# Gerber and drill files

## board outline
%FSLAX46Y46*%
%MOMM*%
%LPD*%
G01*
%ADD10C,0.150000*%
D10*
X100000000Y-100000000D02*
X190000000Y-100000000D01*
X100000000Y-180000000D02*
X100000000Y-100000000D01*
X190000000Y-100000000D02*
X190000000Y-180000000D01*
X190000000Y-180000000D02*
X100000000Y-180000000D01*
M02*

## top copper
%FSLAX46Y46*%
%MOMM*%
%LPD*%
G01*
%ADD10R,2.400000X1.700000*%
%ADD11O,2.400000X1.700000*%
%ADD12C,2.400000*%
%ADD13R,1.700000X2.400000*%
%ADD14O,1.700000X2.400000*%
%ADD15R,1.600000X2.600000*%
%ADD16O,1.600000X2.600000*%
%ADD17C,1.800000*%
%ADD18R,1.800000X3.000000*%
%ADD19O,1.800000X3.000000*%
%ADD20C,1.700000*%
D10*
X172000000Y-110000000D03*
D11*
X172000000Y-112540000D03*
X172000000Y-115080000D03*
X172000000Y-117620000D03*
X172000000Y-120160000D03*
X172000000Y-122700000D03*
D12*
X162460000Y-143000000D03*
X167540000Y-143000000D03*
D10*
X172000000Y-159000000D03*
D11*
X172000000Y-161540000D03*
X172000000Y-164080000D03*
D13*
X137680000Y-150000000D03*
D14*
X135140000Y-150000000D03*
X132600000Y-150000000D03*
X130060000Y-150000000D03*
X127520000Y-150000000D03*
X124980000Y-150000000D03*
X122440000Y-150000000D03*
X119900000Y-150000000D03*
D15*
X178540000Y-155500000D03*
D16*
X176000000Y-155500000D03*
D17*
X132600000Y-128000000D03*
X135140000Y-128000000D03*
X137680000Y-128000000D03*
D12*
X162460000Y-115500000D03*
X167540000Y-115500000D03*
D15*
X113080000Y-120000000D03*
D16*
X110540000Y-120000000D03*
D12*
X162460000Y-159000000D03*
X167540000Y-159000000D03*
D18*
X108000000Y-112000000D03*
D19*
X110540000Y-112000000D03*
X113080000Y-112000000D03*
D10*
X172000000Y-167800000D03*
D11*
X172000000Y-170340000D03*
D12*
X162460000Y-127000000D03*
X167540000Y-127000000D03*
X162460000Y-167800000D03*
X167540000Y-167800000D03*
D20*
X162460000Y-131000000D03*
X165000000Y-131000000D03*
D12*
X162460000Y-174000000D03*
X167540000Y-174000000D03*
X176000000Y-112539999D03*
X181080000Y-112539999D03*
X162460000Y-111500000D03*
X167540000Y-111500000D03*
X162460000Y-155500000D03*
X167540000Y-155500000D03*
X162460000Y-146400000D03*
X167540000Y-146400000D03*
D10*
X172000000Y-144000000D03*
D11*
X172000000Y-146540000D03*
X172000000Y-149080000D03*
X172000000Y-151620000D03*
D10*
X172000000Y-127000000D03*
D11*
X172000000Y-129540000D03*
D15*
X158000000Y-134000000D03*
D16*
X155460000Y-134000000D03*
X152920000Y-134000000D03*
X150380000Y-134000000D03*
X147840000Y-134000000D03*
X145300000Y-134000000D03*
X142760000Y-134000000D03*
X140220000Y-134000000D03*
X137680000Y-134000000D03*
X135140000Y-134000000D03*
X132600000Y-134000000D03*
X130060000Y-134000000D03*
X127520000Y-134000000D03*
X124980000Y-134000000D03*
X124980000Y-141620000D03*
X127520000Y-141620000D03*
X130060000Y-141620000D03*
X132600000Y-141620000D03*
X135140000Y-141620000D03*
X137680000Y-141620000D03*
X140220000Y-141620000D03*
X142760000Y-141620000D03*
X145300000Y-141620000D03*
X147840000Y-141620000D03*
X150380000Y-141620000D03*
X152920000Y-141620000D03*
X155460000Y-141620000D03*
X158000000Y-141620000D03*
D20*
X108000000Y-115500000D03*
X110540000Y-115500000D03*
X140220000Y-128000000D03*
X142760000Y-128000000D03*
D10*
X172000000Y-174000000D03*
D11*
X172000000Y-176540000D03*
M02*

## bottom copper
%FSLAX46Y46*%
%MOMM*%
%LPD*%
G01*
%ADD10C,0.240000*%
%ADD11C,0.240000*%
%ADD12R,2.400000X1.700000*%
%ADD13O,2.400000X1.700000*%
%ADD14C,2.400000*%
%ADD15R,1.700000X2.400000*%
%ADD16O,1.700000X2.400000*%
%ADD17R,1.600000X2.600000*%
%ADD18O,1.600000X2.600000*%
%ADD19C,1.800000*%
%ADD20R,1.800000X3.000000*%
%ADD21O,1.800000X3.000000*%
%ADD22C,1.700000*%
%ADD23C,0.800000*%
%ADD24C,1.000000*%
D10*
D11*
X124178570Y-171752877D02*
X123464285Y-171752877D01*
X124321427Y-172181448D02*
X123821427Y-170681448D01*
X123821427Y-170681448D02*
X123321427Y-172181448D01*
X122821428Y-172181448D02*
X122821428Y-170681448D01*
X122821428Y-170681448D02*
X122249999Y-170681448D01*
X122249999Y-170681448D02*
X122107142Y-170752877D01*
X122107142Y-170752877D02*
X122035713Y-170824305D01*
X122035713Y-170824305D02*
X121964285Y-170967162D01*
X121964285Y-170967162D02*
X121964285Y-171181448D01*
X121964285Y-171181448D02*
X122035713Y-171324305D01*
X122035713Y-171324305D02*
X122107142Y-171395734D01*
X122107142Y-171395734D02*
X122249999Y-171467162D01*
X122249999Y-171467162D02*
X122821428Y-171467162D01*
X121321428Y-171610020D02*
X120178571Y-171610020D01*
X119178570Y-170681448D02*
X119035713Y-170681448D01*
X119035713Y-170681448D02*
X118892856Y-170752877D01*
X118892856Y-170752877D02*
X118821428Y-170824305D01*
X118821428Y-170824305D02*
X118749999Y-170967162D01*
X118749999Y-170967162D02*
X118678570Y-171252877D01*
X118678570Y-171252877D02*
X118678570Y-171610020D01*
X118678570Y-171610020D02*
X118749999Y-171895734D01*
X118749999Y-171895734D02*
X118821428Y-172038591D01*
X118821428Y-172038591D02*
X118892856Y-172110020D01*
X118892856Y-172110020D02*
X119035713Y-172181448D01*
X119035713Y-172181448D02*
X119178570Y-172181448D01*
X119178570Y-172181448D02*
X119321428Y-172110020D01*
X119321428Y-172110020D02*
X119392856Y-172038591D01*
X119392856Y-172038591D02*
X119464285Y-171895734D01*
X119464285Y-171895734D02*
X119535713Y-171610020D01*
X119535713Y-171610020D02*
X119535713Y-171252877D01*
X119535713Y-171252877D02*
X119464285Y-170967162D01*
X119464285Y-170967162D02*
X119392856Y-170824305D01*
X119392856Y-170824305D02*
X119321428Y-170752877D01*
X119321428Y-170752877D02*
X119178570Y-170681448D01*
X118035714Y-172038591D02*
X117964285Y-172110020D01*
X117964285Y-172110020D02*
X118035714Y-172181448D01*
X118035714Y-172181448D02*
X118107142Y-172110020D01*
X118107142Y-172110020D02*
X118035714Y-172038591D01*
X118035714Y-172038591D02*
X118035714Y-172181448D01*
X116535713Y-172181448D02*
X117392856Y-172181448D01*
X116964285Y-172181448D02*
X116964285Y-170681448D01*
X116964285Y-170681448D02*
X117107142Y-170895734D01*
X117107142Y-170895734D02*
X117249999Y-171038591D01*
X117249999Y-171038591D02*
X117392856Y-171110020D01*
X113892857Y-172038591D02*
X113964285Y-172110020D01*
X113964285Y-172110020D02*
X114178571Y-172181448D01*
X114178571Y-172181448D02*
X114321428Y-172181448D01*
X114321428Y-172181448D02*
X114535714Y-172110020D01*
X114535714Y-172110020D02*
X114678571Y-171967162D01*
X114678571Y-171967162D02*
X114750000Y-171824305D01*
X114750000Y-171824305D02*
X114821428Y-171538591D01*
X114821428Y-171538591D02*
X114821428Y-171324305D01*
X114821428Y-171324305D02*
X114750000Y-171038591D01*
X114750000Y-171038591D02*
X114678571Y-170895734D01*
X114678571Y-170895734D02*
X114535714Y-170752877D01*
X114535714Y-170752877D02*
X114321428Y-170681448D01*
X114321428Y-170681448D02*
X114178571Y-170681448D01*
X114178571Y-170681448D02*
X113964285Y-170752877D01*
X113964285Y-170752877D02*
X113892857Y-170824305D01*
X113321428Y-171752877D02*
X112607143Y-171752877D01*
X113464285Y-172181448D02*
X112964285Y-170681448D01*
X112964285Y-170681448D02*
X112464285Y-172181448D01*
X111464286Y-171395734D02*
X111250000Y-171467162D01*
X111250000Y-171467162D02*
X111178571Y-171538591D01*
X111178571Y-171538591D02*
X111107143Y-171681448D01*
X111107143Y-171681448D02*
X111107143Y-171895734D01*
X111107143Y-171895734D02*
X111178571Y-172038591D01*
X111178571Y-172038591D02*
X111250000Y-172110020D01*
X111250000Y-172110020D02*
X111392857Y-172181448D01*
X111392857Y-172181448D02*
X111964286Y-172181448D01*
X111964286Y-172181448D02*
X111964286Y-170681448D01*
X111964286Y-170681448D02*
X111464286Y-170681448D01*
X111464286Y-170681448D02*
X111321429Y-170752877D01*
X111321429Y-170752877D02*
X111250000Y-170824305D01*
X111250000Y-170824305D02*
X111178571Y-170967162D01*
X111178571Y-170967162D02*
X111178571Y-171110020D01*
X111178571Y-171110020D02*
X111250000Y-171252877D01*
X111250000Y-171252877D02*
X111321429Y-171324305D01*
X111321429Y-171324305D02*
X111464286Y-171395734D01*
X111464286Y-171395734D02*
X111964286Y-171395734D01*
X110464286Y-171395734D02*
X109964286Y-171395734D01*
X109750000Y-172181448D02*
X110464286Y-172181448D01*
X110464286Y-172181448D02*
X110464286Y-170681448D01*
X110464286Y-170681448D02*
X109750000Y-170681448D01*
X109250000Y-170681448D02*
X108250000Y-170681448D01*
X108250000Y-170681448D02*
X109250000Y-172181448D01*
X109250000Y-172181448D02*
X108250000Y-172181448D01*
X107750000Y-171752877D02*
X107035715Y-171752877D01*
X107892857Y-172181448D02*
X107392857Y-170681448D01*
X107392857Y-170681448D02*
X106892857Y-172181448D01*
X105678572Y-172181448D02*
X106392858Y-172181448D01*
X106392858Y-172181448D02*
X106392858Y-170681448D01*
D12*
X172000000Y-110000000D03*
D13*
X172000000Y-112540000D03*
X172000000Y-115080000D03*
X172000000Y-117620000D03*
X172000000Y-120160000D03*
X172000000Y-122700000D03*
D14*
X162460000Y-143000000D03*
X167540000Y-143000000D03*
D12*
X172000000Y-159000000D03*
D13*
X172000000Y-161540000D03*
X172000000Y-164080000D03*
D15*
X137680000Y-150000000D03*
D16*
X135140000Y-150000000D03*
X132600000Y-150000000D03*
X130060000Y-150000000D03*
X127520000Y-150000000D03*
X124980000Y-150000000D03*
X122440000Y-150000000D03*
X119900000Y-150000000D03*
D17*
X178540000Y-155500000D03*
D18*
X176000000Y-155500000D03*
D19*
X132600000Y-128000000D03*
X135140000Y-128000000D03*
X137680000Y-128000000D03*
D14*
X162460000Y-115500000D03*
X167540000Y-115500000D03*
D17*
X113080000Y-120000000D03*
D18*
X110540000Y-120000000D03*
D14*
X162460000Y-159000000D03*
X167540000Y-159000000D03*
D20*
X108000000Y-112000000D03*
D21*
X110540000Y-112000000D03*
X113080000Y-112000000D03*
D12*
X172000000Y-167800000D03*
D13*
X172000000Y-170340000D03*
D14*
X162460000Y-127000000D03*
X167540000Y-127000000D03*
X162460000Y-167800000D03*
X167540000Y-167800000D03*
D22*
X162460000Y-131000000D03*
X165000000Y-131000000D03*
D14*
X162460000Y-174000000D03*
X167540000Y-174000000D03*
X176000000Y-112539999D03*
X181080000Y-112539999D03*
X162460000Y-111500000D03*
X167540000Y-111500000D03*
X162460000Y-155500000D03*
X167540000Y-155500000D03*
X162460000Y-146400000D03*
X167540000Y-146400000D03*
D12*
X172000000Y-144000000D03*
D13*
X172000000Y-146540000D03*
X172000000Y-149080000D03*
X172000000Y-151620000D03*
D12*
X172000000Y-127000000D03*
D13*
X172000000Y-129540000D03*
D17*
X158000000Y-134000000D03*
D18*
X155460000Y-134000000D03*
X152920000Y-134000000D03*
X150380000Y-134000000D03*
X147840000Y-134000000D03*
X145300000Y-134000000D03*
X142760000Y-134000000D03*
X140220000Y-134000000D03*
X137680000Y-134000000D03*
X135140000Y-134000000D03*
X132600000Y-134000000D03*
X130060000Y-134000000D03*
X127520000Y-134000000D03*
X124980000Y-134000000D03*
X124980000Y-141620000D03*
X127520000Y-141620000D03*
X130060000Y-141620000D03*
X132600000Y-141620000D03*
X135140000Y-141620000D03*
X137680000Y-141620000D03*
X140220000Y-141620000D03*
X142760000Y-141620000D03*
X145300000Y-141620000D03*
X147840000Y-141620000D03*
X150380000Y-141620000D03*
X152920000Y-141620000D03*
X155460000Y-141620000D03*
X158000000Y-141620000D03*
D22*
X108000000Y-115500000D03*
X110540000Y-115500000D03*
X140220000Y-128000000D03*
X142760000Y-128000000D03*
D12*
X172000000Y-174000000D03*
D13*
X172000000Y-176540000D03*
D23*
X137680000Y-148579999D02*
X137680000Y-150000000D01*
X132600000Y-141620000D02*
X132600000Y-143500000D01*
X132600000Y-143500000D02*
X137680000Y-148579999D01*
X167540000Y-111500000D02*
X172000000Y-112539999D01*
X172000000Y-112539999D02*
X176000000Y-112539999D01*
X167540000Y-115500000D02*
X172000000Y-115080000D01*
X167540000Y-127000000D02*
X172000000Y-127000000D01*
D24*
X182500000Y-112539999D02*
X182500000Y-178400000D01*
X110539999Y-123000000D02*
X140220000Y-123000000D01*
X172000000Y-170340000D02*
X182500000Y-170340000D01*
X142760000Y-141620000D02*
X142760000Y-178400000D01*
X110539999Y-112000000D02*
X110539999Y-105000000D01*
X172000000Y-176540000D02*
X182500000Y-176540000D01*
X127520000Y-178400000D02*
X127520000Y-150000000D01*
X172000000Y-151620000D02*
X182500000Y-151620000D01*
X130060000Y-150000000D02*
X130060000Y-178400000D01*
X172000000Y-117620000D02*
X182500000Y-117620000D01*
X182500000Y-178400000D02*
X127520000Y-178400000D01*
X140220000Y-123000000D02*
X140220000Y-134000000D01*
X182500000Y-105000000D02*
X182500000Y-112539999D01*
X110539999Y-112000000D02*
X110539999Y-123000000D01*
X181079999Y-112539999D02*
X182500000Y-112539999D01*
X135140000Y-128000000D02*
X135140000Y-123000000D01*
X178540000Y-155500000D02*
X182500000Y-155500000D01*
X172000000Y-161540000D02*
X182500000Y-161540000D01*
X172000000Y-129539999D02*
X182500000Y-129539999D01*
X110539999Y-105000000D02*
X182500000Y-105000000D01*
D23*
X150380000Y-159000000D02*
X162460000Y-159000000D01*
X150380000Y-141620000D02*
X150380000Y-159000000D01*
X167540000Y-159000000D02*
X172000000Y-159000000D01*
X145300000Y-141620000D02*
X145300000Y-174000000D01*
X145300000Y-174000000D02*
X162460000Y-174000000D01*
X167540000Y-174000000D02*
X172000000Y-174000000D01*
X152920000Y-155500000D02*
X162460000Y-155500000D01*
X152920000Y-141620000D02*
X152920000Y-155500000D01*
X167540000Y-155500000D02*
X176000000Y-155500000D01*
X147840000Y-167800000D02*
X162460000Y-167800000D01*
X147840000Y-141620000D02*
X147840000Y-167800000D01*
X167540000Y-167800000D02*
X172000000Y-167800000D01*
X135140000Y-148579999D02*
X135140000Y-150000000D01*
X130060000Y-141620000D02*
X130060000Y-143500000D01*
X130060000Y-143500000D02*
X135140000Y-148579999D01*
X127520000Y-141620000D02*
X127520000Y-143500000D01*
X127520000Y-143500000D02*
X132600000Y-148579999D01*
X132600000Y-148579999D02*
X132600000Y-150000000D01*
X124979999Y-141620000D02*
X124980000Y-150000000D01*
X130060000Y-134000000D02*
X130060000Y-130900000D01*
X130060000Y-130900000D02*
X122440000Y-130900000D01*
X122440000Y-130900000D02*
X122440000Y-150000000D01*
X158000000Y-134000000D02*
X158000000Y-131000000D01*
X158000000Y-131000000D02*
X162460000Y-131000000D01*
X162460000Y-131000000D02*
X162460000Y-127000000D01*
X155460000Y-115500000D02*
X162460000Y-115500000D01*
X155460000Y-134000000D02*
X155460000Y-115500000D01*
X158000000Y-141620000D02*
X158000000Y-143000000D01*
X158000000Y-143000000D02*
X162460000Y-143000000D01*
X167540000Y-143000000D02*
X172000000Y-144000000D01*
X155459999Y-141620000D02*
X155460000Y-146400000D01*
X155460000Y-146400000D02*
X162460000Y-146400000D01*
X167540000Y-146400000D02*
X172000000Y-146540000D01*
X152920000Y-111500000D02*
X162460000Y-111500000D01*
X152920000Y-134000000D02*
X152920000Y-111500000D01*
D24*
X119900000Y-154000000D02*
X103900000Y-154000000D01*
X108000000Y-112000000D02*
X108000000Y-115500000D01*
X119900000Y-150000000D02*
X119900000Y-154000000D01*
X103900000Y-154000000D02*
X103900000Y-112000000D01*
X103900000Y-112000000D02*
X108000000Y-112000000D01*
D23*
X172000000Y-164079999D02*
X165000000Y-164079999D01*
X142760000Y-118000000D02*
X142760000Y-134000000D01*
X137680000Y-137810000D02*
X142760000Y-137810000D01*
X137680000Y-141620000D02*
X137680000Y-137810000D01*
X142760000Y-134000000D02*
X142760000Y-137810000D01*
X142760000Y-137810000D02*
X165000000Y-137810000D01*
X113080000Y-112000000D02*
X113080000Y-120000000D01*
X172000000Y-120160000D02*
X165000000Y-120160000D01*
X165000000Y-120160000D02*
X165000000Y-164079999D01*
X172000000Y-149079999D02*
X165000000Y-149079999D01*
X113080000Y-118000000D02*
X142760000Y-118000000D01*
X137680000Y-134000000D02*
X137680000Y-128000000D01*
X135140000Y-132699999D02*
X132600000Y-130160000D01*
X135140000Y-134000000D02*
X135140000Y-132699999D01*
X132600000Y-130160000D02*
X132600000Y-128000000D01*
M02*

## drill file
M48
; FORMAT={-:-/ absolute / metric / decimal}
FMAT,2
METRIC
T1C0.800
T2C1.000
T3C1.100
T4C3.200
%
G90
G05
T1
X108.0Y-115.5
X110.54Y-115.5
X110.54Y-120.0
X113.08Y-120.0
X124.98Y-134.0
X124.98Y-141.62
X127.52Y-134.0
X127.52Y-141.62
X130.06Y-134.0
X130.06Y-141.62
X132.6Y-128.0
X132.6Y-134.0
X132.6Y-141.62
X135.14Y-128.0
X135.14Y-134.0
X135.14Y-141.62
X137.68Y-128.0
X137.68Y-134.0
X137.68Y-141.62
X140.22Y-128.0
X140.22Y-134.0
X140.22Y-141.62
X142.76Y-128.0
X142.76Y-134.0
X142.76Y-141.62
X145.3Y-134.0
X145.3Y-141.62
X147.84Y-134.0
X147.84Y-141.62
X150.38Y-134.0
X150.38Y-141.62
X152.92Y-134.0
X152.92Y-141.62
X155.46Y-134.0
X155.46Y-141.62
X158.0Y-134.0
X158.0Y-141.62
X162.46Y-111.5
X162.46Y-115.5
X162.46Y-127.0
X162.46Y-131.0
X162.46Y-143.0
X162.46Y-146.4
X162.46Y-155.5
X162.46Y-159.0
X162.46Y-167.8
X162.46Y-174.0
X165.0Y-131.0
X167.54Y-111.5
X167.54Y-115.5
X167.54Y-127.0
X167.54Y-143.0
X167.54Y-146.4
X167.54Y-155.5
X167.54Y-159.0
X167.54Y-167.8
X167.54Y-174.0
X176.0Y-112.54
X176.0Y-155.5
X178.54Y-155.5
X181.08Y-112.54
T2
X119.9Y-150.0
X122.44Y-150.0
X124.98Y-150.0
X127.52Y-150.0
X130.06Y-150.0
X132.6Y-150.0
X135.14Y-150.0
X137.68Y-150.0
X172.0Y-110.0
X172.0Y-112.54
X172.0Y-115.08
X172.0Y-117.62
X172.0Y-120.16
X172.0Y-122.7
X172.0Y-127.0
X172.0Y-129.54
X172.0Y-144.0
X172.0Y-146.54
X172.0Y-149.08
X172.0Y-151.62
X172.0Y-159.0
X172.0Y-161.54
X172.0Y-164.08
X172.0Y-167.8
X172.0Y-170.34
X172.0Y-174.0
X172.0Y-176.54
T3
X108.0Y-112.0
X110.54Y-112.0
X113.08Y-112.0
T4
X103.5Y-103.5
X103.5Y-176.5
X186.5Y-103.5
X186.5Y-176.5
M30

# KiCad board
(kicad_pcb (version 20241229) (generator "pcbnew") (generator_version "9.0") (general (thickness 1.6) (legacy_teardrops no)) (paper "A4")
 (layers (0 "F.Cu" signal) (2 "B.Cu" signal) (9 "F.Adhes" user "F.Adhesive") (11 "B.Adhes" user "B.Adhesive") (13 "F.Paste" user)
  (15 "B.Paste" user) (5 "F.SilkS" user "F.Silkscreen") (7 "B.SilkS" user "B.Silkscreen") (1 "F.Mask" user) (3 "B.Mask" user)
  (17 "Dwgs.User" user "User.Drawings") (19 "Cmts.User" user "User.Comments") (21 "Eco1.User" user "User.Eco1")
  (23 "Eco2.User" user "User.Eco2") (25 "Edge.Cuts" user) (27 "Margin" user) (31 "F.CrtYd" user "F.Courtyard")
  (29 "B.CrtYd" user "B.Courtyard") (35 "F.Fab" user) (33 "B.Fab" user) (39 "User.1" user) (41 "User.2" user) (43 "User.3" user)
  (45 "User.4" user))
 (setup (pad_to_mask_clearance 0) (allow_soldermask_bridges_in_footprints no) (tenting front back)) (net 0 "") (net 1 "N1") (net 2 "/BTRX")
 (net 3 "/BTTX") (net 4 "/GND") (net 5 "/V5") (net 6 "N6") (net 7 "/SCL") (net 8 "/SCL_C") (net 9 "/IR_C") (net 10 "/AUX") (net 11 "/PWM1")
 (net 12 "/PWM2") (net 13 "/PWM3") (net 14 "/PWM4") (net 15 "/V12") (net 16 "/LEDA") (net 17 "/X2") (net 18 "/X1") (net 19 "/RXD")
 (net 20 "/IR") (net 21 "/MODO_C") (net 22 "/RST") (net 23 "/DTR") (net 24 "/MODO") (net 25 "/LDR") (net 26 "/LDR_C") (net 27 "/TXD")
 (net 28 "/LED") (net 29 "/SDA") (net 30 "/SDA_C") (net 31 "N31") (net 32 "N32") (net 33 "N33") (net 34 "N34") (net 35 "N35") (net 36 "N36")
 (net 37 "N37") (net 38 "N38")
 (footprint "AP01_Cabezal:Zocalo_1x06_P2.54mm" (layer "F.Cu") (at 172 110)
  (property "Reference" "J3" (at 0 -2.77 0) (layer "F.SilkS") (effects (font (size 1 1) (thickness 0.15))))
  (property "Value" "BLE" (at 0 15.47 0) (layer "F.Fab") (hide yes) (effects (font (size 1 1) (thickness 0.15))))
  (pad "1" thru_hole rect (at 0 0) (size 2.4 1.7) (drill 1) (layers "B.Cu" "B.Mask") (remove_unused_layers no) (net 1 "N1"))
  (pad "2" thru_hole oval (at 0 2.54) (size 2.4 1.7) (drill 1) (layers "B.Cu" "B.Mask") (remove_unused_layers no) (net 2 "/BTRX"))
  (pad "3" thru_hole oval (at 0 5.08) (size 2.4 1.7) (drill 1) (layers "B.Cu" "B.Mask") (remove_unused_layers no) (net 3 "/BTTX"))
  (pad "4" thru_hole oval (at 0 7.62) (size 2.4 1.7) (drill 1) (layers "B.Cu" "B.Mask") (remove_unused_layers no) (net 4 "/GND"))
  (pad "5" thru_hole oval (at 0 10.16) (size 2.4 1.7) (drill 1) (layers "B.Cu" "B.Mask") (remove_unused_layers no) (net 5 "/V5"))
  (pad "6" thru_hole oval (at 0 12.7) (size 2.4 1.7) (drill 1) (layers "B.Cu" "B.Mask") (remove_unused_layers no) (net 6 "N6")))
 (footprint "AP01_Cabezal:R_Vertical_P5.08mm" (layer "F.Cu") (at 162.46 143)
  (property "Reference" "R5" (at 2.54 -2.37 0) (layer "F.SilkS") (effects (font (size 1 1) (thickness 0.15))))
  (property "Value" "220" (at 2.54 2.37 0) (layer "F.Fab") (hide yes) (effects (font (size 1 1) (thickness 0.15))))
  (pad "1" thru_hole circle (at 0 0) (size 2.4 2.4) (drill 0.8) (layers "B.Cu" "B.Mask") (remove_unused_layers no) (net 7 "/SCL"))
  (pad "2" thru_hole circle (at 5.08 0) (size 2.4 2.4) (drill 0.8) (layers "B.Cu" "B.Mask") (remove_unused_layers no) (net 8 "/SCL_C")))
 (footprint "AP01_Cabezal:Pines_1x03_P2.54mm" (layer "F.Cu") (at 172 159)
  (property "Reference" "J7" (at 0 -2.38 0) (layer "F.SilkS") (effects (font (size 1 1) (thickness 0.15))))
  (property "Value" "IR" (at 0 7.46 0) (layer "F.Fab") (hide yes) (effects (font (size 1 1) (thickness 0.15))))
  (pad "1" thru_hole rect (at 0 0) (size 2.4 1.7) (drill 1) (layers "B.Cu" "B.Mask") (remove_unused_layers no) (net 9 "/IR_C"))
  (pad "2" thru_hole oval (at 0 2.54) (size 2.4 1.7) (drill 1) (layers "B.Cu" "B.Mask") (remove_unused_layers no) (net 4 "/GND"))
  (pad "3" thru_hole oval (at 0 5.08) (size 2.4 1.7) (drill 1) (layers "B.Cu" "B.Mask") (remove_unused_layers no) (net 5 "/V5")))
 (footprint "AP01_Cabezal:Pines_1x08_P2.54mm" (layer "F.Cu") (at 137.68 150 -90)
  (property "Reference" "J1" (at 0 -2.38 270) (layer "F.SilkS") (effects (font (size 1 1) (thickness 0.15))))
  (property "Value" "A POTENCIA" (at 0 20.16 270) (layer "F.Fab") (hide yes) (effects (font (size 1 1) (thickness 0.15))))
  (pad "1" thru_hole rect (at 0 0 270) (size 2.4 1.7) (drill 1) (layers "B.Cu" "B.Mask") (remove_unused_layers no) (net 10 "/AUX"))
  (pad "2" thru_hole oval (at 0 2.54 270) (size 2.4 1.7) (drill 1) (layers "B.Cu" "B.Mask") (remove_unused_layers no) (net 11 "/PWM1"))
  (pad "3" thru_hole oval (at 0 5.08 270) (size 2.4 1.7) (drill 1) (layers "B.Cu" "B.Mask") (remove_unused_layers no) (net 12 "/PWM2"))
  (pad "4" thru_hole oval (at 0 7.62 270) (size 2.4 1.7) (drill 1) (layers "B.Cu" "B.Mask") (remove_unused_layers no) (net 4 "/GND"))
  (pad "5" thru_hole oval (at 0 10.16 270) (size 2.4 1.7) (drill 1) (layers "B.Cu" "B.Mask") (remove_unused_layers no) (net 4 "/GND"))
  (pad "6" thru_hole oval (at 0 12.7 270) (size 2.4 1.7) (drill 1) (layers "B.Cu" "B.Mask") (remove_unused_layers no) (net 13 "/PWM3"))
  (pad "7" thru_hole oval (at 0 15.24 270) (size 2.4 1.7) (drill 1) (layers "B.Cu" "B.Mask") (remove_unused_layers no) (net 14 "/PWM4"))
  (pad "8" thru_hole oval (at 0 17.78 270) (size 2.4 1.7) (drill 1) (layers "B.Cu" "B.Mask") (remove_unused_layers no) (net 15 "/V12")))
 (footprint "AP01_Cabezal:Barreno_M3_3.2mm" (layer "F.Cu") (at 103.5 176.5)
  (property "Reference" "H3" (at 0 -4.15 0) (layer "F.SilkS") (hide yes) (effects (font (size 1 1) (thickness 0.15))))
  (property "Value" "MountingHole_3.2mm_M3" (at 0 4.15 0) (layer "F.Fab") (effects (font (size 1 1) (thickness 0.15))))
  (pad "" np_thru_hole circle (at 0 0) (size 3.2 3.2) (drill 3.2) (layers "*.Cu" "*.Mask")))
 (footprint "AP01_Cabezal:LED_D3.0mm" (layer "F.Cu") (at 178.54 155.5 180)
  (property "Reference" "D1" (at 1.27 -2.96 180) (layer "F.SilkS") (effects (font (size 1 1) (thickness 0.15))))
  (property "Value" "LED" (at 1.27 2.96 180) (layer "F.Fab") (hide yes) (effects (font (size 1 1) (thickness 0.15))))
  (pad "1" thru_hole rect (at 0 0 180) (size 1.6 2.6) (drill 0.8) (layers "B.Cu" "B.Mask") (remove_unused_layers no) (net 4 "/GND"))
  (pad "2" thru_hole oval (at 2.54 0 180) (size 1.6 2.6) (drill 0.8) (layers "B.Cu" "B.Mask") (remove_unused_layers no) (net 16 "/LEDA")))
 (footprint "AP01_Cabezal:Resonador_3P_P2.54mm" (layer "F.Cu") (at 132.6 128)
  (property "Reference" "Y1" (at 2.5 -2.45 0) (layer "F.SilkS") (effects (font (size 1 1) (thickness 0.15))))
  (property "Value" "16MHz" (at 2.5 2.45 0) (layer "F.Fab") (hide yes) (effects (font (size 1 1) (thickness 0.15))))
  (pad "1" thru_hole circle (at 0 0) (size 1.8 1.8) (drill 0.8) (layers "B.Cu" "B.Mask") (remove_unused_layers no) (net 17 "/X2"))
  (pad "2" thru_hole circle (at 2.54 0) (size 1.8 1.8) (drill 0.8) (layers "B.Cu" "B.Mask") (remove_unused_layers no) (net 4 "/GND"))
  (pad "3" thru_hole circle (at 5.08 0) (size 1.8 1.8) (drill 0.8) (layers "B.Cu" "B.Mask") (remove_unused_layers no) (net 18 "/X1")))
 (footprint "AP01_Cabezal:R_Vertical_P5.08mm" (layer "F.Cu") (at 162.46 115.5)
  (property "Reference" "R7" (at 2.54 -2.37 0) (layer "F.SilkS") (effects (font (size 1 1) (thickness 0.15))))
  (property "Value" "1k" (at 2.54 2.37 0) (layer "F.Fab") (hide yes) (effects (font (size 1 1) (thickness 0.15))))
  (pad "1" thru_hole circle (at 0 0) (size 2.4 2.4) (drill 0.8) (layers "B.Cu" "B.Mask") (remove_unused_layers no) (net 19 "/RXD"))
  (pad "2" thru_hole circle (at 5.08 0) (size 2.4 2.4) (drill 0.8) (layers "B.Cu" "B.Mask") (remove_unused_layers no) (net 3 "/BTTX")))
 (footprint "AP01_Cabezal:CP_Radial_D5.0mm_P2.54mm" (layer "F.Cu") (at 113.08 120 180)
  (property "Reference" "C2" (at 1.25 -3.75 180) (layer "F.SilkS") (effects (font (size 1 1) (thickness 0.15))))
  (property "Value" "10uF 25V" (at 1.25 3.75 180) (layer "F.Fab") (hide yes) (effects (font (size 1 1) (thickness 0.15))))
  (pad "1" thru_hole rect (at 0 0 180) (size 1.6 2.6) (drill 0.8) (layers "B.Cu" "B.Mask") (remove_unused_layers no) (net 5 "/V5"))
  (pad "2" thru_hole oval (at 2.54 0 180) (size 1.6 2.6) (drill 0.8) (layers "B.Cu" "B.Mask") (remove_unused_layers no) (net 4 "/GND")))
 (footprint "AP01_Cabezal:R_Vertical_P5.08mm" (layer "F.Cu") (at 162.46 159)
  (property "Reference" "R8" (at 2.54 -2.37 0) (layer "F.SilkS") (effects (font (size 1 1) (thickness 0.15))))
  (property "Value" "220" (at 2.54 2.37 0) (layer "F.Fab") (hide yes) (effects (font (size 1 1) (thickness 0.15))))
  (pad "1" thru_hole circle (at 0 0) (size 2.4 2.4) (drill 0.8) (layers "B.Cu" "B.Mask") (remove_unused_layers no) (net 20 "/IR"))
  (pad "2" thru_hole circle (at 5.08 0) (size 2.4 2.4) (drill 0.8) (layers "B.Cu" "B.Mask") (remove_unused_layers no) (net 9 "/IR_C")))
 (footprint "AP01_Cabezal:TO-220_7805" (layer "F.Cu") (at 108 112)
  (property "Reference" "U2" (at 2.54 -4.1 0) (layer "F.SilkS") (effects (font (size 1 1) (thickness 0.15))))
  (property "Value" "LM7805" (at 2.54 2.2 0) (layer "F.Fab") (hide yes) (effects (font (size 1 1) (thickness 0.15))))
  (pad "1" thru_hole rect (at 0 0) (size 1.8 3) (drill 1.1) (layers "B.Cu" "B.Mask") (remove_unused_layers no) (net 15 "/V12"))
  (pad "2" thru_hole oval (at 2.54 0) (size 1.8 3) (drill 1.1) (layers "B.Cu" "B.Mask") (remove_unused_layers no) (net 4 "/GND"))
  (pad "3" thru_hole oval (at 5.08 0) (size 1.8 3) (drill 1.1) (layers "B.Cu" "B.Mask") (remove_unused_layers no) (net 5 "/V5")))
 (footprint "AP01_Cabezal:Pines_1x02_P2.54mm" (layer "F.Cu") (at 172 167.8)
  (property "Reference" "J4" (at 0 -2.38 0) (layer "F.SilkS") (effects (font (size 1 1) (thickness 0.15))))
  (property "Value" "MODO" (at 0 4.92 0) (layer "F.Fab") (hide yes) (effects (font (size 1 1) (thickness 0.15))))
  (pad "1" thru_hole rect (at 0 0) (size 2.4 1.7) (drill 1) (layers "B.Cu" "B.Mask") (remove_unused_layers no) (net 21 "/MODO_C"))
  (pad "2" thru_hole oval (at 0 2.54) (size 2.4 1.7) (drill 1) (layers "B.Cu" "B.Mask") (remove_unused_layers no) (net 4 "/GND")))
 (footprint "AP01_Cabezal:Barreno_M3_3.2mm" (layer "F.Cu") (at 103.5 103.5)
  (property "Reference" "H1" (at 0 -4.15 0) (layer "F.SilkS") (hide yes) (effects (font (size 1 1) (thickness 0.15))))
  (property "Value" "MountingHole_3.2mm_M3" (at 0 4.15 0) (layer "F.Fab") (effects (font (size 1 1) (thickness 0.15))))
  (pad "" np_thru_hole circle (at 0 0) (size 3.2 3.2) (drill 3.2) (layers "*.Cu" "*.Mask")))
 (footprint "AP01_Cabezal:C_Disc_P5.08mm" (layer "F.Cu") (at 162.46 127)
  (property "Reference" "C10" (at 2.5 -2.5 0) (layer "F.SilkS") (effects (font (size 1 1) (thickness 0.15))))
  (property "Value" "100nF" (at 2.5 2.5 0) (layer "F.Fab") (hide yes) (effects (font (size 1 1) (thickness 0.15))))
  (pad "1" thru_hole circle (at 0 0) (size 2.4 2.4) (drill 0.8) (layers "B.Cu" "B.Mask") (remove_unused_layers no) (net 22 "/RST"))
  (pad "2" thru_hole circle (at 5.08 0) (size 2.4 2.4) (drill 0.8) (layers "B.Cu" "B.Mask") (remove_unused_layers no) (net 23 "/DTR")))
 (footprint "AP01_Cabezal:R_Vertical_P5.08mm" (layer "F.Cu") (at 162.46 167.8)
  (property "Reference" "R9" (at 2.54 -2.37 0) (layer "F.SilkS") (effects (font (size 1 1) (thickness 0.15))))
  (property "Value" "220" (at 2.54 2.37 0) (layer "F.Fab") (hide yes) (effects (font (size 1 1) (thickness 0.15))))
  (pad "1" thru_hole circle (at 0 0) (size 2.4 2.4) (drill 0.8) (layers "B.Cu" "B.Mask") (remove_unused_layers no) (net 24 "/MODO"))
  (pad "2" thru_hole circle (at 5.08 0) (size 2.4 2.4) (drill 0.8) (layers "B.Cu" "B.Mask") (remove_unused_layers no) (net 21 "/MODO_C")))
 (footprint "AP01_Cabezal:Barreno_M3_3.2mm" (layer "F.Cu") (at 186.5 176.5)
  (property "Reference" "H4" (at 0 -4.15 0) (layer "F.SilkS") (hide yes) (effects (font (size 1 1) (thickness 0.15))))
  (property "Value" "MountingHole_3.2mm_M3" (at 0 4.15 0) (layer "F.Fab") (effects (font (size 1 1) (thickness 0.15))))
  (pad "" np_thru_hole circle (at 0 0) (size 3.2 3.2) (drill 3.2) (layers "*.Cu" "*.Mask")))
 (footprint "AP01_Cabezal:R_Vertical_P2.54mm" (layer "F.Cu") (at 162.46 131)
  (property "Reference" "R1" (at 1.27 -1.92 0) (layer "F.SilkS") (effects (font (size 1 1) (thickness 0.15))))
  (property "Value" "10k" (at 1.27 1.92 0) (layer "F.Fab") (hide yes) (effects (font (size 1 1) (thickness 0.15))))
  (pad "1" thru_hole circle (at 0 0) (size 1.7 1.7) (drill 0.8) (layers "B.Cu" "B.Mask") (remove_unused_layers no) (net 22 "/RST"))
  (pad "2" thru_hole circle (at 2.54 0) (size 1.7 1.7) (drill 0.8) (layers "B.Cu" "B.Mask") (remove_unused_layers no) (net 5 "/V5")))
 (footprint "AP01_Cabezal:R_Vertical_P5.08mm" (layer "F.Cu") (at 162.46 174)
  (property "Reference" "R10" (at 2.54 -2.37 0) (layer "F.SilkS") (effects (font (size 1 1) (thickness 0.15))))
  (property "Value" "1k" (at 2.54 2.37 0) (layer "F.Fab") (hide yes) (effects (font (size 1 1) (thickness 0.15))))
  (pad "1" thru_hole circle (at 0 0) (size 2.4 2.4) (drill 0.8) (layers "B.Cu" "B.Mask") (remove_unused_layers no) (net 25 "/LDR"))
  (pad "2" thru_hole circle (at 5.08 0) (size 2.4 2.4) (drill 0.8) (layers "B.Cu" "B.Mask") (remove_unused_layers no) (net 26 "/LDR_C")))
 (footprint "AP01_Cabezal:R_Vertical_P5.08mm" (layer "F.Cu") (at 176 112.539999)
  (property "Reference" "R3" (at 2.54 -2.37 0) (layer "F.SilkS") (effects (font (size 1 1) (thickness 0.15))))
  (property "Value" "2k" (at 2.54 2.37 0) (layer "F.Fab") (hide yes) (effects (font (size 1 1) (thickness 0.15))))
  (pad "1" thru_hole circle (at 0 0) (size 2.4 2.4) (drill 0.8) (layers "B.Cu" "B.Mask") (remove_unused_layers no) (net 2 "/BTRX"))
  (pad "2" thru_hole circle (at 5.08 0) (size 2.4 2.4) (drill 0.8) (layers "B.Cu" "B.Mask") (remove_unused_layers no) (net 4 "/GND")))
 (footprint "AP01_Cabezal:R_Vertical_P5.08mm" (layer "F.Cu") (at 162.46 111.5)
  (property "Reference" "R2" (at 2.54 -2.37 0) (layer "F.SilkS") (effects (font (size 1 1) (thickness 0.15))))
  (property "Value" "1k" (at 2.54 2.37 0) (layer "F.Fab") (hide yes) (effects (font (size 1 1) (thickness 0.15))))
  (pad "1" thru_hole circle (at 0 0) (size 2.4 2.4) (drill 0.8) (layers "B.Cu" "B.Mask") (remove_unused_layers no) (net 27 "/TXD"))
  (pad "2" thru_hole circle (at 5.08 0) (size 2.4 2.4) (drill 0.8) (layers "B.Cu" "B.Mask") (remove_unused_layers no) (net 2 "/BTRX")))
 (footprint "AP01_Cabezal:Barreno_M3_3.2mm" (layer "F.Cu") (at 186.5 103.5)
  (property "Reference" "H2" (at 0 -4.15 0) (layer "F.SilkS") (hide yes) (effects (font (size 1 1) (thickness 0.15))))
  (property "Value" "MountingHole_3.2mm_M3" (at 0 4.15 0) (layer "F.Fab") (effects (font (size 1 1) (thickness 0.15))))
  (pad "" np_thru_hole circle (at 0 0) (size 3.2 3.2) (drill 3.2) (layers "*.Cu" "*.Mask")))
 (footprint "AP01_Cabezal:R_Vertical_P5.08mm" (layer "F.Cu") (at 162.46 155.5)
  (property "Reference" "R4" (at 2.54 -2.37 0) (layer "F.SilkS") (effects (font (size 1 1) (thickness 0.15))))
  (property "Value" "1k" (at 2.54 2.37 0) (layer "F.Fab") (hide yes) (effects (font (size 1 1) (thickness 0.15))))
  (pad "1" thru_hole circle (at 0 0) (size 2.4 2.4) (drill 0.8) (layers "B.Cu" "B.Mask") (remove_unused_layers no) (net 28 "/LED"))
  (pad "2" thru_hole circle (at 5.08 0) (size 2.4 2.4) (drill 0.8) (layers "B.Cu" "B.Mask") (remove_unused_layers no) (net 16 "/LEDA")))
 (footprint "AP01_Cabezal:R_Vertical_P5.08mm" (layer "F.Cu") (at 162.46 146.4)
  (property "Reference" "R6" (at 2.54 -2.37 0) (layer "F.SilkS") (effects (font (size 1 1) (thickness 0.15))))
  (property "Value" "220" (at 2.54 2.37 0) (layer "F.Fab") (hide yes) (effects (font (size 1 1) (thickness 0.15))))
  (pad "1" thru_hole circle (at 0 0) (size 2.4 2.4) (drill 0.8) (layers "B.Cu" "B.Mask") (remove_unused_layers no) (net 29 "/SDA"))
  (pad "2" thru_hole circle (at 5.08 0) (size 2.4 2.4) (drill 0.8) (layers "B.Cu" "B.Mask") (remove_unused_layers no) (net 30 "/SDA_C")))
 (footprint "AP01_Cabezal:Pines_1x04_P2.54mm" (layer "F.Cu") (at 172 144)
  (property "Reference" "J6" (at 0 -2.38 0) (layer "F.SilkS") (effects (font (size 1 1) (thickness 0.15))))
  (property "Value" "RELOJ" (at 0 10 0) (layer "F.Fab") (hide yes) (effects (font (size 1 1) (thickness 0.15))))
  (pad "1" thru_hole rect (at 0 0) (size 2.4 1.7) (drill 1) (layers "B.Cu" "B.Mask") (remove_unused_layers no) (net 8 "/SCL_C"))
  (pad "2" thru_hole oval (at 0 2.54) (size 2.4 1.7) (drill 1) (layers "B.Cu" "B.Mask") (remove_unused_layers no) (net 30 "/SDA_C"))
  (pad "3" thru_hole oval (at 0 5.08) (size 2.4 1.7) (drill 1) (layers "B.Cu" "B.Mask") (remove_unused_layers no) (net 5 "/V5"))
  (pad "4" thru_hole oval (at 0 7.62) (size 2.4 1.7) (drill 1) (layers "B.Cu" "B.Mask") (remove_unused_layers no) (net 4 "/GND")))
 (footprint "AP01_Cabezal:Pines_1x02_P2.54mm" (layer "F.Cu") (at 172 127)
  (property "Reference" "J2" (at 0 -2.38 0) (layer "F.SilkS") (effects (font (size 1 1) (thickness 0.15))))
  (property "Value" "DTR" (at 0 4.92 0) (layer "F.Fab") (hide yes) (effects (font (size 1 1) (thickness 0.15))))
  (pad "1" thru_hole rect (at 0 0) (size 2.4 1.7) (drill 1) (layers "B.Cu" "B.Mask") (remove_unused_layers no) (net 23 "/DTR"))
  (pad "2" thru_hole oval (at 0 2.54) (size 2.4 1.7) (drill 1) (layers "B.Cu" "B.Mask") (remove_unused_layers no) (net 4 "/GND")))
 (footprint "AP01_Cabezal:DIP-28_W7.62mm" (layer "F.Cu") (at 158 134 -90)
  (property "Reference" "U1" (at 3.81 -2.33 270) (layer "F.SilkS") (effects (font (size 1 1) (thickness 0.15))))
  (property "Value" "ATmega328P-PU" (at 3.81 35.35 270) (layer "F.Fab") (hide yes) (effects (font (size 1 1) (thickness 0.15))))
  (pad "1" thru_hole rect (at 0 0 270) (size 2.6 1.6) (drill 0.8) (layers "B.Cu" "B.Mask") (remove_unused_layers no) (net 22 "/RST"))
  (pad "2" thru_hole oval (at 0 2.54 270) (size 2.6 1.6) (drill 0.8) (layers "B.Cu" "B.Mask") (remove_unused_layers no) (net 19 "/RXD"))
  (pad "3" thru_hole oval (at 0 5.08 270) (size 2.6 1.6) (drill 0.8) (layers "B.Cu" "B.Mask") (remove_unused_layers no) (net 27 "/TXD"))
  (pad "4" thru_hole oval (at 0 7.62 270) (size 2.6 1.6) (drill 0.8) (layers "B.Cu" "B.Mask") (remove_unused_layers no) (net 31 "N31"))
  (pad "5" thru_hole oval (at 0 10.16 270) (size 2.6 1.6) (drill 0.8) (layers "B.Cu" "B.Mask") (remove_unused_layers no) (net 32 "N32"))
  (pad "6" thru_hole oval (at 0 12.7 270) (size 2.6 1.6) (drill 0.8) (layers "B.Cu" "B.Mask") (remove_unused_layers no) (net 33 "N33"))
  (pad "7" thru_hole oval (at 0 15.24 270) (size 2.6 1.6) (drill 0.8) (layers "B.Cu" "B.Mask") (remove_unused_layers no) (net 5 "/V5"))
  (pad "8" thru_hole oval (at 0 17.78 270) (size 2.6 1.6) (drill 0.8) (layers "B.Cu" "B.Mask") (remove_unused_layers no) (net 4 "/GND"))
  (pad "9" thru_hole oval (at 0 20.32 270) (size 2.6 1.6) (drill 0.8) (layers "B.Cu" "B.Mask") (remove_unused_layers no) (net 18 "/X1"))
  (pad "10" thru_hole oval (at 0 22.86 270) (size 2.6 1.6) (drill 0.8) (layers "B.Cu" "B.Mask") (remove_unused_layers no) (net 17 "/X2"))
  (pad "11" thru_hole oval (at 0 25.4 270) (size 2.6 1.6) (drill 0.8) (layers "B.Cu" "B.Mask") (remove_unused_layers no) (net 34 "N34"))
  (pad "12" thru_hole oval (at 0 27.94 270) (size 2.6 1.6) (drill 0.8) (layers "B.Cu" "B.Mask") (remove_unused_layers no) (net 14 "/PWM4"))
  (pad "13" thru_hole oval (at 0 30.48 270) (size 2.6 1.6) (drill 0.8) (layers "B.Cu" "B.Mask") (remove_unused_layers no) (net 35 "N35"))
  (pad "14" thru_hole oval (at 0 33.02 270) (size 2.6 1.6) (drill 0.8) (layers "B.Cu" "B.Mask") (remove_unused_layers no) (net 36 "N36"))
  (pad "15" thru_hole oval (at 7.62 33.02 270) (size 2.6 1.6) (drill 0.8) (layers "B.Cu" "B.Mask") (remove_unused_layers no)
   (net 13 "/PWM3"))
  (pad "16" thru_hole oval (at 7.62 30.48 270) (size 2.6 1.6) (drill 0.8) (layers "B.Cu" "B.Mask") (remove_unused_layers no)
   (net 12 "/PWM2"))
  (pad "17" thru_hole oval (at 7.62 27.94 270) (size 2.6 1.6) (drill 0.8) (layers "B.Cu" "B.Mask") (remove_unused_layers no)
   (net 11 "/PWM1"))
  (pad "18" thru_hole oval (at 7.62 25.4 270) (size 2.6 1.6) (drill 0.8) (layers "B.Cu" "B.Mask") (remove_unused_layers no) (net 10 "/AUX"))
  (pad "19" thru_hole oval (at 7.62 22.86 270) (size 2.6 1.6) (drill 0.8) (layers "B.Cu" "B.Mask") (remove_unused_layers no) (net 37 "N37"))
  (pad "20" thru_hole oval (at 7.62 20.32 270) (size 2.6 1.6) (drill 0.8) (layers "B.Cu" "B.Mask") (remove_unused_layers no) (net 5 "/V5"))
  (pad "21" thru_hole oval (at 7.62 17.78 270) (size 2.6 1.6) (drill 0.8) (layers "B.Cu" "B.Mask") (remove_unused_layers no) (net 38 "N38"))
  (pad "22" thru_hole oval (at 7.62 15.24 270) (size 2.6 1.6) (drill 0.8) (layers "B.Cu" "B.Mask") (remove_unused_layers no) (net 4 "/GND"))
  (pad "23" thru_hole oval (at 7.62 12.7 270) (size 2.6 1.6) (drill 0.8) (layers "B.Cu" "B.Mask") (remove_unused_layers no) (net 25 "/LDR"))
  (pad "24" thru_hole oval (at 7.62 10.16 270) (size 2.6 1.6) (drill 0.8) (layers "B.Cu" "B.Mask") (remove_unused_layers no)
   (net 24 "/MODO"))
  (pad "25" thru_hole oval (at 7.62 7.62 270) (size 2.6 1.6) (drill 0.8) (layers "B.Cu" "B.Mask") (remove_unused_layers no) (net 20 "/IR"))
  (pad "26" thru_hole oval (at 7.62 5.08 270) (size 2.6 1.6) (drill 0.8) (layers "B.Cu" "B.Mask") (remove_unused_layers no) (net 28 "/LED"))
  (pad "27" thru_hole oval (at 7.62 2.54 270) (size 2.6 1.6) (drill 0.8) (layers "B.Cu" "B.Mask") (remove_unused_layers no) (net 29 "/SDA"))
  (pad "28" thru_hole oval (at 7.62 0 270) (size 2.6 1.6) (drill 0.8) (layers "B.Cu" "B.Mask") (remove_unused_layers no) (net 7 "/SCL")))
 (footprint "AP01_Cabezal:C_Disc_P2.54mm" (layer "F.Cu") (at 108 115.5)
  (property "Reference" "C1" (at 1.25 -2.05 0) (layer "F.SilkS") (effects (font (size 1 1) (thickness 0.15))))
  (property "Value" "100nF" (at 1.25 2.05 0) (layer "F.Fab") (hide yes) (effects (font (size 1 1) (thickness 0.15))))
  (pad "1" thru_hole circle (at 0 0) (size 1.7 1.7) (drill 0.8) (layers "B.Cu" "B.Mask") (remove_unused_layers no) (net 15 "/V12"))
  (pad "2" thru_hole circle (at 2.54 0) (size 1.7 1.7) (drill 0.8) (layers "B.Cu" "B.Mask") (remove_unused_layers no) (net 4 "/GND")))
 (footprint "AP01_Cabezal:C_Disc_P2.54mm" (layer "F.Cu") (at 140.22 128)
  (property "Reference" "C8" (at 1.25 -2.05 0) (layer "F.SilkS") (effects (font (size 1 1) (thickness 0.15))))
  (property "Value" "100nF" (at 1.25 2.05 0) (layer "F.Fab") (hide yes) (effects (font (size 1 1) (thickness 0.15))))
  (pad "1" thru_hole circle (at 0 0) (size 1.7 1.7) (drill 0.8) (layers "B.Cu" "B.Mask") (remove_unused_layers no) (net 4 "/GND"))
  (pad "2" thru_hole circle (at 2.54 0) (size 1.7 1.7) (drill 0.8) (layers "B.Cu" "B.Mask") (remove_unused_layers no) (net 5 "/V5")))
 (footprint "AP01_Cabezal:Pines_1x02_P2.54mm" (layer "F.Cu") (at 172 174)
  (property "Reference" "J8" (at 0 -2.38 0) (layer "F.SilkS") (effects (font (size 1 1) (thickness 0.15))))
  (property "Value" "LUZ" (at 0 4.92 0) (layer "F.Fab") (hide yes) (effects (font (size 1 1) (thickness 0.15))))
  (pad "1" thru_hole rect (at 0 0) (size 2.4 1.7) (drill 1) (layers "B.Cu" "B.Mask") (remove_unused_layers no) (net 26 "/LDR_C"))
  (pad "2" thru_hole oval (at 0 2.54) (size 2.4 1.7) (drill 1) (layers "B.Cu" "B.Mask") (remove_unused_layers no) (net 4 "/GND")))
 (gr_line (start 100 100) (end 190 100) (stroke (width 0.15) (type default)) (layer "Edge.Cuts"))
 (gr_line (start 100 180) (end 100 100) (stroke (width 0.15) (type default)) (layer "Edge.Cuts"))
 (gr_line (start 190 100) (end 190 180) (stroke (width 0.15) (type default)) (layer "Edge.Cuts"))
 (gr_line (start 190 180) (end 100 180) (stroke (width 0.15) (type default)) (layer "Edge.Cuts"))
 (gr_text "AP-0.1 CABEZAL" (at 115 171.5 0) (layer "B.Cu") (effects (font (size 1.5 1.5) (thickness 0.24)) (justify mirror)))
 (segment (start 137.68 148.579999) (end 137.68 150) (width 0.8) (layer "B.Cu") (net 10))
 (segment (start 132.6 141.62) (end 132.6 143.5) (width 0.8) (layer "B.Cu") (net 10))
 (segment (start 132.6 143.5) (end 137.68 148.579999) (width 0.8) (layer "B.Cu") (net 10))
 (segment (start 167.54 111.5) (end 172 112.539999) (width 0.8) (layer "B.Cu") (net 2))
 (segment (start 172 112.539999) (end 176 112.539999) (width 0.8) (layer "B.Cu") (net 2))
 (segment (start 167.54 115.5) (end 172 115.08) (width 0.8) (layer "B.Cu") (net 3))
 (segment (start 167.54 127) (end 172 127) (width 0.8) (layer "B.Cu") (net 23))
 (segment (start 182.5 112.539999) (end 182.5 178.4) (width 1) (layer "B.Cu") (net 4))
 (segment (start 110.539999 123) (end 140.22 123) (width 1) (layer "B.Cu") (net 4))
 (segment (start 172 170.34) (end 182.5 170.34) (width 1) (layer "B.Cu") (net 4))
 (segment (start 142.76 141.62) (end 142.76 178.4) (width 1) (layer "B.Cu") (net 4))
 (segment (start 110.539999 112) (end 110.539999 105) (width 1) (layer "B.Cu") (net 4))
 (segment (start 172 176.54) (end 182.5 176.54) (width 1) (layer "B.Cu") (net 4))
 (segment (start 127.52 178.4) (end 127.52 150) (width 1) (layer "B.Cu") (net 4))
 (segment (start 172 151.62) (end 182.5 151.62) (width 1) (layer "B.Cu") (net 4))
 (segment (start 130.06 150) (end 130.06 178.4) (width 1) (layer "B.Cu") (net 4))
 (segment (start 172 117.62) (end 182.5 117.62) (width 1) (layer "B.Cu") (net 4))
 (segment (start 182.5 178.4) (end 127.52 178.4) (width 1) (layer "B.Cu") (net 4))
 (segment (start 140.22 123) (end 140.22 134) (width 1) (layer "B.Cu") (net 4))
 (segment (start 182.5 105) (end 182.5 112.539999) (width 1) (layer "B.Cu") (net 4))
 (segment (start 110.539999 112) (end 110.539999 123) (width 1) (layer "B.Cu") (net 4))
 (segment (start 181.079999 112.539999) (end 182.5 112.539999) (width 1) (layer "B.Cu") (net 4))
 (segment (start 135.14 128) (end 135.14 123) (width 1) (layer "B.Cu") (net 4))
 (segment (start 178.54 155.5) (end 182.5 155.5) (width 1) (layer "B.Cu") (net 4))
 (segment (start 172 161.54) (end 182.5 161.54) (width 1) (layer "B.Cu") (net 4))
 (segment (start 172 129.539999) (end 182.5 129.539999) (width 1) (layer "B.Cu") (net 4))
 (segment (start 110.539999 105) (end 182.5 105) (width 1) (layer "B.Cu") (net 4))
 (segment (start 150.38 159) (end 162.46 159) (width 0.8) (layer "B.Cu") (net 20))
 (segment (start 150.38 141.62) (end 150.38 159) (width 0.8) (layer "B.Cu") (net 20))
 (segment (start 167.54 159) (end 172 159) (width 0.8) (layer "B.Cu") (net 9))
 (segment (start 145.3 141.62) (end 145.3 174) (width 0.8) (layer "B.Cu") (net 25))
 (segment (start 145.3 174) (end 162.46 174) (width 0.8) (layer "B.Cu") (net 25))
 (segment (start 167.54 174) (end 172 174) (width 0.8) (layer "B.Cu") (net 26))
 (segment (start 152.92 155.5) (end 162.46 155.5) (width 0.8) (layer "B.Cu") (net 28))
 (segment (start 152.92 141.62) (end 152.92 155.5) (width 0.8) (layer "B.Cu") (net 28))
 (segment (start 167.54 155.5) (end 176 155.5) (width 0.8) (layer "B.Cu") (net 16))
 (segment (start 147.84 167.8) (end 162.46 167.8) (width 0.8) (layer "B.Cu") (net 24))
 (segment (start 147.84 141.62) (end 147.84 167.8) (width 0.8) (layer "B.Cu") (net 24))
 (segment (start 167.54 167.8) (end 172 167.8) (width 0.8) (layer "B.Cu") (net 21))
 (segment (start 135.14 148.579999) (end 135.14 150) (width 0.8) (layer "B.Cu") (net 11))
 (segment (start 130.06 141.62) (end 130.06 143.5) (width 0.8) (layer "B.Cu") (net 11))
 (segment (start 130.06 143.5) (end 135.14 148.579999) (width 0.8) (layer "B.Cu") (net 11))
 (segment (start 127.52 141.62) (end 127.52 143.5) (width 0.8) (layer "B.Cu") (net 12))
 (segment (start 127.52 143.5) (end 132.6 148.579999) (width 0.8) (layer "B.Cu") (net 12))
 (segment (start 132.6 148.579999) (end 132.6 150) (width 0.8) (layer "B.Cu") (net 12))
 (segment (start 124.979999 141.62) (end 124.98 150) (width 0.8) (layer "B.Cu") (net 13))
 (segment (start 130.06 134) (end 130.06 130.9) (width 0.8) (layer "B.Cu") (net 14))
 (segment (start 130.06 130.9) (end 122.44 130.9) (width 0.8) (layer "B.Cu") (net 14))
 (segment (start 122.44 130.9) (end 122.44 150) (width 0.8) (layer "B.Cu") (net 14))
 (segment (start 158 134) (end 158 131) (width 0.8) (layer "B.Cu") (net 22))
 (segment (start 158 131) (end 162.46 131) (width 0.8) (layer "B.Cu") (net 22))
 (segment (start 162.46 131) (end 162.46 127) (width 0.8) (layer "B.Cu") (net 22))
 (segment (start 155.46 115.5) (end 162.46 115.5) (width 0.8) (layer "B.Cu") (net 19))
 (segment (start 155.46 134) (end 155.46 115.5) (width 0.8) (layer "B.Cu") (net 19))
 (segment (start 158 141.62) (end 158 143) (width 0.8) (layer "B.Cu") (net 7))
 (segment (start 158 143) (end 162.46 143) (width 0.8) (layer "B.Cu") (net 7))
 (segment (start 167.54 143) (end 172 144) (width 0.8) (layer "B.Cu") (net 8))
 (segment (start 155.459999 141.62) (end 155.46 146.4) (width 0.8) (layer "B.Cu") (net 29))
 (segment (start 155.46 146.4) (end 162.46 146.4) (width 0.8) (layer "B.Cu") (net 29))
 (segment (start 167.54 146.4) (end 172 146.54) (width 0.8) (layer "B.Cu") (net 30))
 (segment (start 152.92 111.5) (end 162.46 111.5) (width 0.8) (layer "B.Cu") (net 27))
 (segment (start 152.92 134) (end 152.92 111.5) (width 0.8) (layer "B.Cu") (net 27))
 (segment (start 119.9 154) (end 103.9 154) (width 1) (layer "B.Cu") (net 15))
 (segment (start 108 112) (end 108 115.5) (width 1) (layer "B.Cu") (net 15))
 (segment (start 119.9 150) (end 119.9 154) (width 1) (layer "B.Cu") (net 15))
 (segment (start 103.9 154) (end 103.9 112) (width 1) (layer "B.Cu") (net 15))
 (segment (start 103.9 112) (end 108 112) (width 1) (layer "B.Cu") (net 15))
 (segment (start 172 164.079999) (end 165 164.079999) (width 0.8) (layer "B.Cu") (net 5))
 (segment (start 142.76 118) (end 142.76 134) (width 0.8) (layer "B.Cu") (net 5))
 (segment (start 137.68 137.81) (end 142.76 137.81) (width 0.8) (layer "B.Cu") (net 5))
 (segment (start 137.68 141.62) (end 137.68 137.81) (width 0.8) (layer "B.Cu") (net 5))
 (segment (start 142.76 134) (end 142.76 137.81) (width 0.8) (layer "B.Cu") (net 5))
 (segment (start 142.76 137.81) (end 165 137.81) (width 0.8) (layer "B.Cu") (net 5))
 (segment (start 113.08 112) (end 113.08 120) (width 0.8) (layer "B.Cu") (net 5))
 (segment (start 172 120.16) (end 165 120.16) (width 0.8) (layer "B.Cu") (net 5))
 (segment (start 165 120.16) (end 165 164.079999) (width 0.8) (layer "B.Cu") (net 5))
 (segment (start 172 149.079999) (end 165 149.079999) (width 0.8) (layer "B.Cu") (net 5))
 (segment (start 113.08 118) (end 142.76 118) (width 0.8) (layer "B.Cu") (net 5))
 (segment (start 137.68 134) (end 137.68 128) (width 0.8) (layer "B.Cu") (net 18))
 (segment (start 135.14 132.699999) (end 132.6 130.16) (width 0.8) (layer "B.Cu") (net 17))
 (segment (start 135.14 134) (end 135.14 132.699999) (width 0.8) (layer "B.Cu") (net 17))
 (segment (start 132.6 130.16) (end 132.6 128) (width 0.8) (layer "B.Cu") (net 17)))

